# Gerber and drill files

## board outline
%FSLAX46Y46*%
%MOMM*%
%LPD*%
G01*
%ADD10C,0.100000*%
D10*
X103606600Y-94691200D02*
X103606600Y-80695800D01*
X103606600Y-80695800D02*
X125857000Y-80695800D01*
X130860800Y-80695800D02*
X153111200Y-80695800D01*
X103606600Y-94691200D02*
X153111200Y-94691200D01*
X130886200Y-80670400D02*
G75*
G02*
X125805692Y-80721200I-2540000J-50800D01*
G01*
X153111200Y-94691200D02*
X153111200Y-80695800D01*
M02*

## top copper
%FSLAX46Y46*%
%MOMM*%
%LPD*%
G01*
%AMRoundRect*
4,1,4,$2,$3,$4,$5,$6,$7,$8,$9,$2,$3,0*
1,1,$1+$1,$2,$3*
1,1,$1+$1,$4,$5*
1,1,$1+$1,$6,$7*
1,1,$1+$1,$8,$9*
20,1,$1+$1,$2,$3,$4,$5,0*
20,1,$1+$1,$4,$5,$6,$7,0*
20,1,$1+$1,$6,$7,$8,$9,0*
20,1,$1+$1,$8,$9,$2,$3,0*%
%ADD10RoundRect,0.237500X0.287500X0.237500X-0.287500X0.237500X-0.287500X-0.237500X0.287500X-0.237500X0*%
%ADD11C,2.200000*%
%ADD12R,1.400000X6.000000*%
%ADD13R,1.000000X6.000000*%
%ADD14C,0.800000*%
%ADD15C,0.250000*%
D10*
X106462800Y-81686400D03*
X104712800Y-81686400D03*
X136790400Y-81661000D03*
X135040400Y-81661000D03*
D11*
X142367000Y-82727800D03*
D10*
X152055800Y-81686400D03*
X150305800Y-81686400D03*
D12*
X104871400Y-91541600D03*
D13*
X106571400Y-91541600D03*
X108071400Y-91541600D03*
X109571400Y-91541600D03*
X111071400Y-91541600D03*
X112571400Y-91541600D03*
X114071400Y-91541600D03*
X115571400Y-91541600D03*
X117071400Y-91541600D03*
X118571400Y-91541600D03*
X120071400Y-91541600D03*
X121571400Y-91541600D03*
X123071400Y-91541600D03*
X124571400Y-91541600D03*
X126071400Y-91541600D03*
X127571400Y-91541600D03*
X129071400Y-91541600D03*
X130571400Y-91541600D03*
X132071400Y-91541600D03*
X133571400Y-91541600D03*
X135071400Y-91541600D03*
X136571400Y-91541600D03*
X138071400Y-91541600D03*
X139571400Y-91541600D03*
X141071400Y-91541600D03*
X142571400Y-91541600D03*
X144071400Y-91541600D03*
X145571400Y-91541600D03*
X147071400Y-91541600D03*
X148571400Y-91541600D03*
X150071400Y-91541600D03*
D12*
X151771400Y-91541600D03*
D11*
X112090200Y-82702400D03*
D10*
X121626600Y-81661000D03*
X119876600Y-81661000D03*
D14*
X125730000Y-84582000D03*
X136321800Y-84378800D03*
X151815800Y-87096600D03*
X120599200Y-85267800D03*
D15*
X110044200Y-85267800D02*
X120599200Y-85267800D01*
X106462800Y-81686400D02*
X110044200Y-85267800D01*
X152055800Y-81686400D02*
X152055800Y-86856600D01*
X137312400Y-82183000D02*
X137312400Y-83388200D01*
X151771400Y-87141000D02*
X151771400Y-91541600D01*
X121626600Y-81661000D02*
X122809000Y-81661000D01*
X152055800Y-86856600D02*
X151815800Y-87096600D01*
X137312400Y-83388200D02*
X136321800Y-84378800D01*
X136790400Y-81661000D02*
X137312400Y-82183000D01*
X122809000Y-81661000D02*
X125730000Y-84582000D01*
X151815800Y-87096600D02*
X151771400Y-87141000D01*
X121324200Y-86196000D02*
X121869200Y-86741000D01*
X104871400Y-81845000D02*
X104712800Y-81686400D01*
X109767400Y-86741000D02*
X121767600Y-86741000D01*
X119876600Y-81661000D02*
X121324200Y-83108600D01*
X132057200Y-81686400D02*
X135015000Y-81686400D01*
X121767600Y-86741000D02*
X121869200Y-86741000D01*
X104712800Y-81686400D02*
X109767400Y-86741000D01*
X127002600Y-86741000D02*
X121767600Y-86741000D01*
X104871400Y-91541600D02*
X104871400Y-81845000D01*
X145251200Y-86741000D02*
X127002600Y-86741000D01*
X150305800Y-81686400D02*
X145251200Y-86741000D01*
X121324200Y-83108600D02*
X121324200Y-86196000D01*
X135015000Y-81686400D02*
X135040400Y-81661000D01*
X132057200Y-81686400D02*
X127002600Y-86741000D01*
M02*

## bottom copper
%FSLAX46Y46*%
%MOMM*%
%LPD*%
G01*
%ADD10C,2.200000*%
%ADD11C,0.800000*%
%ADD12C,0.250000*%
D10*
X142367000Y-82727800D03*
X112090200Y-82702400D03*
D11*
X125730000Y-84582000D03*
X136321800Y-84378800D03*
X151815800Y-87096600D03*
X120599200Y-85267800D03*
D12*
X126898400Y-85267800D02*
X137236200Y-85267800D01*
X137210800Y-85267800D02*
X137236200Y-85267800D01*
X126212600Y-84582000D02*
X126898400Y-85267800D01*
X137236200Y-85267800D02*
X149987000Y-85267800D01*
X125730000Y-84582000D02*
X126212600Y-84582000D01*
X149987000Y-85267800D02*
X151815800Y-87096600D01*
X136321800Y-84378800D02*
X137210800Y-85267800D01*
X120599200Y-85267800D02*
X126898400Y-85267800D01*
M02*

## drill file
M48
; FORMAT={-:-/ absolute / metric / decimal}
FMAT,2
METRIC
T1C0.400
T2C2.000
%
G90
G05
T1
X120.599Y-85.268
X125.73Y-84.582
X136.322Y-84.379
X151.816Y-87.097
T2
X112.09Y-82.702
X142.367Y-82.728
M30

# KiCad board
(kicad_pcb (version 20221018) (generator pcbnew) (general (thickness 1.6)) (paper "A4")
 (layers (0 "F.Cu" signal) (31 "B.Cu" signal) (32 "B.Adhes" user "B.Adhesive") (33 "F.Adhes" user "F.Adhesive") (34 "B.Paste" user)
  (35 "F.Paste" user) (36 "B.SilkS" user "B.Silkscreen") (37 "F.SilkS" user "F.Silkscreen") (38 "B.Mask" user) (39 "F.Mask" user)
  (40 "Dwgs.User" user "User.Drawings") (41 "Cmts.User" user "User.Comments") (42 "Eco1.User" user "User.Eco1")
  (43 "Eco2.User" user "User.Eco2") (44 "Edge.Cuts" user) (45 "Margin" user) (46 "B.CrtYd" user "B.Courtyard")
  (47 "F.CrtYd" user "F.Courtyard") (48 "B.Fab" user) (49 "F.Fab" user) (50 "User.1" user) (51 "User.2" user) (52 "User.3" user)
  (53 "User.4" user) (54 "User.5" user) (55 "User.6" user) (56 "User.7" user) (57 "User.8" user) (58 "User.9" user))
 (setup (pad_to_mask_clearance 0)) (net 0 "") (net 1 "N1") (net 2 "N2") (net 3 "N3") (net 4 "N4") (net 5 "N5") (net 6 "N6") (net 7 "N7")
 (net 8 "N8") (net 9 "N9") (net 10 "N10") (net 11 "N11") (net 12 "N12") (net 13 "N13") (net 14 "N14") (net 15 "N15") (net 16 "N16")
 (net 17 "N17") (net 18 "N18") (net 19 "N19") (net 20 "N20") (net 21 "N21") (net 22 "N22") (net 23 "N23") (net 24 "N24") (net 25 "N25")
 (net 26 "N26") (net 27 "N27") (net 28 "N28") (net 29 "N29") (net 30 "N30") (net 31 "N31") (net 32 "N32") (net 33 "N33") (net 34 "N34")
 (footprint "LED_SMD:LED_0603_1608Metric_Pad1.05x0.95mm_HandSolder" (layer "F.Cu") (at 105.5878 81.6864 180)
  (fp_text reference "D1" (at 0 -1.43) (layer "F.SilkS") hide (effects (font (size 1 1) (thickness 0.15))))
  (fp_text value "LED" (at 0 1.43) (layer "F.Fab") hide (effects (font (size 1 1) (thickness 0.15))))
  (pad "1" smd roundrect (at -0.875 0 180) (size 1.05 0.95) (layers "F.Cu" "F.Paste" "F.Mask") (roundrect_rratio 0.25) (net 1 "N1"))
  (pad "2" smd roundrect (at 0.875 0 180) (size 1.05 0.95) (layers "F.Cu" "F.Paste" "F.Mask") (roundrect_rratio 0.25) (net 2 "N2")))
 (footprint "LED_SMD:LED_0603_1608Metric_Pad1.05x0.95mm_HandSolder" (layer "F.Cu") (at 135.9154 81.661 180)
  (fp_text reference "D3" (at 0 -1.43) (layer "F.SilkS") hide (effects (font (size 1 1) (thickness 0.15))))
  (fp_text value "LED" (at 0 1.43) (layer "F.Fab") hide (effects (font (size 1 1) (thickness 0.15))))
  (pad "1" smd roundrect (at -0.875 0 180) (size 1.05 0.95) (layers "F.Cu" "F.Paste" "F.Mask") (roundrect_rratio 0.25) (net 1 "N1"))
  (pad "2" smd roundrect (at 0.875 0 180) (size 1.05 0.95) (layers "F.Cu" "F.Paste" "F.Mask") (roundrect_rratio 0.25) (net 2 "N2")))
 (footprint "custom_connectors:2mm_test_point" (layer "F.Cu") (at 142.367 82.73796)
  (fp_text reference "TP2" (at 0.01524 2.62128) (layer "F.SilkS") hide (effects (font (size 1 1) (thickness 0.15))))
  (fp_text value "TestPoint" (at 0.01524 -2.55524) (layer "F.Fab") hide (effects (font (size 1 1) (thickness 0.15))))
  (pad "1" thru_hole circle (at 0 -0.01016) (size 2.2 2.2) (drill 2) (layers "*.Cu" "*.Mask") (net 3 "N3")))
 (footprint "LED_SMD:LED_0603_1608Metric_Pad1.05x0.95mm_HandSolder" (layer "F.Cu") (at 151.1808 81.6864 180)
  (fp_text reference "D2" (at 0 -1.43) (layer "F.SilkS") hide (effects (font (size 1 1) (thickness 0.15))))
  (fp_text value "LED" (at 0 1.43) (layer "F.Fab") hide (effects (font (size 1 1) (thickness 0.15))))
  (pad "1" smd roundrect (at -0.875 0 180) (size 1.05 0.95) (layers "F.Cu" "F.Paste" "F.Mask") (roundrect_rratio 0.25) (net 1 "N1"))
  (pad "2" smd roundrect (at 0.875 0 180) (size 1.05 0.95) (layers "F.Cu" "F.Paste" "F.Mask") (roundrect_rratio 0.25) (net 2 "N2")))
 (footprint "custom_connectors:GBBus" (layer "F.Cu") (at 104.1714 88.5416)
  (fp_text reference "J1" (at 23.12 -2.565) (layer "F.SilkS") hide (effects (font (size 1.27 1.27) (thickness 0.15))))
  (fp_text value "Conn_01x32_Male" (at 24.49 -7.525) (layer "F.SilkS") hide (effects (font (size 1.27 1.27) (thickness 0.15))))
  (pad "1" smd rect (at 0.7 3 180) (size 1.4 6) (layers "F.Cu" "F.Paste" "F.Mask") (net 2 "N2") (solder_mask_margin 0.0508))
  (pad "2" smd rect (at 2.4 3) (size 1 6) (layers "F.Cu" "F.Paste" "F.Mask") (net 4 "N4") (solder_mask_margin 0.0508))
  (pad "3" smd rect (at 3.9 3 180) (size 1 6) (layers "F.Cu" "F.Paste" "F.Mask") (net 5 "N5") (solder_mask_margin 0.0508))
  (pad "4" smd rect (at 5.4 3 180) (size 1 6) (layers "F.Cu" "F.Paste" "F.Mask") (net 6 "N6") (solder_mask_margin 0.0508))
  (pad "5" smd rect (at 6.9 3) (size 1 6) (layers "F.Cu" "F.Paste" "F.Mask") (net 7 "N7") (solder_mask_margin 0.0508))
  (pad "6" smd rect (at 8.4 3) (size 1 6) (layers "F.Cu" "F.Paste" "F.Mask") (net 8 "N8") (solder_mask_margin 0.0508))
  (pad "7" smd rect (at 9.9 3) (size 1 6) (layers "F.Cu" "F.Paste" "F.Mask") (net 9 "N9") (solder_mask_margin 0.0508))
  (pad "8" smd rect (at 11.4 3) (size 1 6) (layers "F.Cu" "F.Paste" "F.Mask") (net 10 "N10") (solder_mask_margin 0.0508))
  (pad "9" smd rect (at 12.9 3) (size 1 6) (layers "F.Cu" "F.Paste" "F.Mask") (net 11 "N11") (solder_mask_margin 0.0508))
  (pad "10" smd rect (at 14.4 3) (size 1 6) (layers "F.Cu" "F.Paste" "F.Mask") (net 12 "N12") (solder_mask_margin 0.0508))
  (pad "11" smd rect (at 15.9 3) (size 1 6) (layers "F.Cu" "F.Paste" "F.Mask") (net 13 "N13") (solder_mask_margin 0.0508))
  (pad "12" smd rect (at 17.4 3) (size 1 6) (layers "F.Cu" "F.Paste" "F.Mask") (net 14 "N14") (solder_mask_margin 0.0508))
  (pad "13" smd rect (at 18.9 3) (size 1 6) (layers "F.Cu" "F.Paste" "F.Mask") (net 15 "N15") (solder_mask_margin 0.0508))
  (pad "14" smd rect (at 20.4 3) (size 1 6) (layers "F.Cu" "F.Paste" "F.Mask") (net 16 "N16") (solder_mask_margin 0.0508))
  (pad "15" smd rect (at 21.9 3) (size 1 6) (layers "F.Cu" "F.Paste" "F.Mask") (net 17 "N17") (solder_mask_margin 0.0508))
  (pad "16" smd rect (at 23.4 3) (size 1 6) (layers "F.Cu" "F.Paste" "F.Mask") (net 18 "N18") (solder_mask_margin 0.0508))
  (pad "17" smd rect (at 24.9 3) (size 1 6) (layers "F.Cu" "F.Paste" "F.Mask") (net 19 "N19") (solder_mask_margin 0.0508))
  (pad "18" smd rect (at 26.4 3) (size 1 6) (layers "F.Cu" "F.Paste" "F.Mask") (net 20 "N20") (solder_mask_margin 0.0508))
  (pad "19" smd rect (at 27.9 3) (size 1 6) (layers "F.Cu" "F.Paste" "F.Mask") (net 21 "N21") (solder_mask_margin 0.0508))
  (pad "20" smd rect (at 29.4 3) (size 1 6) (layers "F.Cu" "F.Paste" "F.Mask") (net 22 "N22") (solder_mask_margin 0.0508))
  (pad "21" smd rect (at 30.9 3) (size 1 6) (layers "F.Cu" "F.Paste" "F.Mask") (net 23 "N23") (solder_mask_margin 0.0508))
  (pad "22" smd rect (at 32.4 3) (size 1 6) (layers "F.Cu" "F.Paste" "F.Mask") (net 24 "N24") (solder_mask_margin 0.0508))
  (pad "23" smd rect (at 33.9 3) (size 1 6) (layers "F.Cu" "F.Paste" "F.Mask") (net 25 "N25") (solder_mask_margin 0.0508))
  (pad "24" smd rect (at 35.4 3) (size 1 6) (layers "F.Cu" "F.Paste" "F.Mask") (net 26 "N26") (solder_mask_margin 0.0508))
  (pad "25" smd rect (at 36.9 3) (size 1 6) (layers "F.Cu" "F.Paste" "F.Mask") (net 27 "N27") (solder_mask_margin 0.0508))
  (pad "26" smd rect (at 38.4 3) (size 1 6) (layers "F.Cu" "F.Paste" "F.Mask") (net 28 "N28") (solder_mask_margin 0.0508))
  (pad "27" smd rect (at 39.9 3) (size 1 6) (layers "F.Cu" "F.Paste" "F.Mask") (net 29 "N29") (solder_mask_margin 0.0508))
  (pad "28" smd rect (at 41.4 3) (size 1 6) (layers "F.Cu" "F.Paste" "F.Mask") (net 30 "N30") (solder_mask_margin 0.0508))
  (pad "29" smd rect (at 42.9 3) (size 1 6) (layers "F.Cu" "F.Paste" "F.Mask") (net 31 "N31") (solder_mask_margin 0.0508))
  (pad "30" smd rect (at 44.4 3) (size 1 6) (layers "F.Cu" "F.Paste" "F.Mask") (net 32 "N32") (solder_mask_margin 0.0508))
  (pad "31" smd rect (at 45.9 3) (size 1 6) (layers "F.Cu" "F.Paste" "F.Mask") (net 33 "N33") (solder_mask_margin 0.0508))
  (pad "32" smd rect (at 47.6 3 180) (size 1.4 6) (layers "F.Cu" "F.Paste" "F.Mask") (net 1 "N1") (solder_mask_margin 0.0508)))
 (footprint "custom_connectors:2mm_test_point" (layer "F.Cu") (at 112.0902 82.71256)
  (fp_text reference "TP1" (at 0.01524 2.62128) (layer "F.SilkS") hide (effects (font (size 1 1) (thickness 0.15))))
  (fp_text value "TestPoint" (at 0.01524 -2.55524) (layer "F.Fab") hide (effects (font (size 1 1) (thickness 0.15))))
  (pad "1" thru_hole circle (at 0 -0.01016) (size 2.2 2.2) (drill 2) (layers "*.Cu" "*.Mask") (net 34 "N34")))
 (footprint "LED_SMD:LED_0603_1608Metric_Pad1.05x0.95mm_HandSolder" (layer "F.Cu") (at 120.7516 81.661 180)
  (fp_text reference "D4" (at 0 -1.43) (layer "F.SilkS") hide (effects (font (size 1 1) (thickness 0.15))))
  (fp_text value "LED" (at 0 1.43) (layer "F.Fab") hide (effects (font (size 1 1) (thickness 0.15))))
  (pad "1" smd roundrect (at -0.875 0 180) (size 1.05 0.95) (layers "F.Cu" "F.Paste" "F.Mask") (roundrect_rratio 0.25) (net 1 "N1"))
  (pad "2" smd roundrect (at 0.875 0 180) (size 1.05 0.95) (layers "F.Cu" "F.Paste" "F.Mask") (roundrect_rratio 0.25) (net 2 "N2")))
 (gr_line (start 103.6066 94.6912) (end 103.6066 80.6958) (stroke (width 0.1) (type solid)) (layer "Edge.Cuts"))
 (gr_line (start 103.6066 80.6958) (end 125.857 80.6958) (stroke (width 0.1) (type solid)) (layer "Edge.Cuts"))
 (gr_line (start 130.8608 80.6958) (end 153.1112 80.6958) (stroke (width 0.1) (type solid)) (layer "Edge.Cuts"))
 (gr_line (start 103.6066 94.6912) (end 153.1112 94.6912) (stroke (width 0.1) (type solid)) (layer "Edge.Cuts"))
 (gr_arc (start 130.8862 80.6704) (mid 128.371602 83.26158) (end 125.805694 80.7212) (stroke (width 0.1) (type solid)) (layer "Edge.Cuts"))
 (gr_line (start 153.1112 94.6912) (end 153.1112 80.6958) (stroke (width 0.1) (type solid)) (layer "Edge.Cuts"))
 (segment (start 110.0442 85.2678) (end 120.5992 85.2678) (width 0.25) (layer "F.Cu") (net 1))
 (segment (start 106.4628 81.6864) (end 110.0442 85.2678) (width 0.25) (layer "F.Cu") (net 1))
 (segment (start 152.0558 81.6864) (end 152.0558 86.8566) (width 0.25) (layer "F.Cu") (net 1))
 (segment (start 137.3124 82.183) (end 137.3124 83.3882) (width 0.25) (layer "F.Cu") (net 1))
 (segment (start 151.7714 87.141) (end 151.7714 91.5416) (width 0.25) (layer "F.Cu") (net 1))
 (segment (start 121.6266 81.661) (end 122.809 81.661) (width 0.25) (layer "F.Cu") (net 1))
 (segment (start 152.0558 86.8566) (end 151.8158 87.0966) (width 0.25) (layer "F.Cu") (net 1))
 (segment (start 137.3124 83.3882) (end 136.3218 84.3788) (width 0.25) (layer "F.Cu") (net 1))
 (segment (start 136.7904 81.661) (end 137.3124 82.183) (width 0.25) (layer "F.Cu") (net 1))
 (segment (start 122.809 81.661) (end 125.73 84.582) (width 0.25) (layer "F.Cu") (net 1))
 (segment (start 151.8158 87.0966) (end 151.7714 87.141) (width 0.25) (layer "F.Cu") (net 1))
 (via (at 125.73 84.582) (size 0.8) (drill 0.4) (layers "F.Cu" "B.Cu") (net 1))
 (via (at 136.3218 84.3788) (size 0.8) (drill 0.4) (layers "F.Cu" "B.Cu") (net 1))
 (via (at 151.8158 87.0966) (size 0.8) (drill 0.4) (layers "F.Cu" "B.Cu") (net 1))
 (via (at 120.5992 85.2678) (size 0.8) (drill 0.4) (layers "F.Cu" "B.Cu") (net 1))
 (segment (start 126.8984 85.2678) (end 137.2362 85.2678) (width 0.25) (layer "B.Cu") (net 1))
 (segment (start 137.2108 85.2678) (end 137.2362 85.2678) (width 0.25) (layer "B.Cu") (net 1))
 (segment (start 126.2126 84.582) (end 126.8984 85.2678) (width 0.25) (layer "B.Cu") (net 1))
 (segment (start 137.2362 85.2678) (end 149.987 85.2678) (width 0.25) (layer "B.Cu") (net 1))
 (segment (start 125.73 84.582) (end 126.2126 84.582) (width 0.25) (layer "B.Cu") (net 1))
 (segment (start 149.987 85.2678) (end 151.8158 87.0966) (width 0.25) (layer "B.Cu") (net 1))
 (segment (start 136.3218 84.3788) (end 137.2108 85.2678) (width 0.25) (layer "B.Cu") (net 1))
 (segment (start 120.5992 85.2678) (end 126.8984 85.2678) (width 0.25) (layer "B.Cu") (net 1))
 (segment (start 121.3242 86.196) (end 121.8692 86.741) (width 0.25) (layer "F.Cu") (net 2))
 (segment (start 104.8714 81.845) (end 104.7128 81.6864) (width 0.25) (layer "F.Cu") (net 2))
 (segment (start 109.7674 86.741) (end 121.7676 86.741) (width 0.25) (layer "F.Cu") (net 2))
 (segment (start 119.8766 81.661) (end 121.3242 83.1086) (width 0.25) (layer "F.Cu") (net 2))
 (segment (start 132.0572 81.6864) (end 135.015 81.6864) (width 0.25) (layer "F.Cu") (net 2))
 (segment (start 121.7676 86.741) (end 121.8692 86.741) (width 0.25) (layer "F.Cu") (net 2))
 (segment (start 104.7128 81.6864) (end 109.7674 86.741) (width 0.25) (layer "F.Cu") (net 2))
 (segment (start 127.0026 86.741) (end 121.7676 86.741) (width 0.25) (layer "F.Cu") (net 2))
 (segment (start 104.8714 91.5416) (end 104.8714 81.845) (width 0.25) (layer "F.Cu") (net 2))
 (segment (start 145.2512 86.741) (end 127.0026 86.741) (width 0.25) (layer "F.Cu") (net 2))
 (segment (start 150.3058 81.6864) (end 145.2512 86.741) (width 0.25) (layer "F.Cu") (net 2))
 (segment (start 121.3242 83.1086) (end 121.3242 86.196) (width 0.25) (layer "F.Cu") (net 2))
 (segment (start 135.015 81.6864) (end 135.0404 81.661) (width 0.25) (layer "F.Cu") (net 2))
 (segment (start 132.0572 81.6864) (end 127.0026 86.741) (width 0.25) (layer "F.Cu") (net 2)))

